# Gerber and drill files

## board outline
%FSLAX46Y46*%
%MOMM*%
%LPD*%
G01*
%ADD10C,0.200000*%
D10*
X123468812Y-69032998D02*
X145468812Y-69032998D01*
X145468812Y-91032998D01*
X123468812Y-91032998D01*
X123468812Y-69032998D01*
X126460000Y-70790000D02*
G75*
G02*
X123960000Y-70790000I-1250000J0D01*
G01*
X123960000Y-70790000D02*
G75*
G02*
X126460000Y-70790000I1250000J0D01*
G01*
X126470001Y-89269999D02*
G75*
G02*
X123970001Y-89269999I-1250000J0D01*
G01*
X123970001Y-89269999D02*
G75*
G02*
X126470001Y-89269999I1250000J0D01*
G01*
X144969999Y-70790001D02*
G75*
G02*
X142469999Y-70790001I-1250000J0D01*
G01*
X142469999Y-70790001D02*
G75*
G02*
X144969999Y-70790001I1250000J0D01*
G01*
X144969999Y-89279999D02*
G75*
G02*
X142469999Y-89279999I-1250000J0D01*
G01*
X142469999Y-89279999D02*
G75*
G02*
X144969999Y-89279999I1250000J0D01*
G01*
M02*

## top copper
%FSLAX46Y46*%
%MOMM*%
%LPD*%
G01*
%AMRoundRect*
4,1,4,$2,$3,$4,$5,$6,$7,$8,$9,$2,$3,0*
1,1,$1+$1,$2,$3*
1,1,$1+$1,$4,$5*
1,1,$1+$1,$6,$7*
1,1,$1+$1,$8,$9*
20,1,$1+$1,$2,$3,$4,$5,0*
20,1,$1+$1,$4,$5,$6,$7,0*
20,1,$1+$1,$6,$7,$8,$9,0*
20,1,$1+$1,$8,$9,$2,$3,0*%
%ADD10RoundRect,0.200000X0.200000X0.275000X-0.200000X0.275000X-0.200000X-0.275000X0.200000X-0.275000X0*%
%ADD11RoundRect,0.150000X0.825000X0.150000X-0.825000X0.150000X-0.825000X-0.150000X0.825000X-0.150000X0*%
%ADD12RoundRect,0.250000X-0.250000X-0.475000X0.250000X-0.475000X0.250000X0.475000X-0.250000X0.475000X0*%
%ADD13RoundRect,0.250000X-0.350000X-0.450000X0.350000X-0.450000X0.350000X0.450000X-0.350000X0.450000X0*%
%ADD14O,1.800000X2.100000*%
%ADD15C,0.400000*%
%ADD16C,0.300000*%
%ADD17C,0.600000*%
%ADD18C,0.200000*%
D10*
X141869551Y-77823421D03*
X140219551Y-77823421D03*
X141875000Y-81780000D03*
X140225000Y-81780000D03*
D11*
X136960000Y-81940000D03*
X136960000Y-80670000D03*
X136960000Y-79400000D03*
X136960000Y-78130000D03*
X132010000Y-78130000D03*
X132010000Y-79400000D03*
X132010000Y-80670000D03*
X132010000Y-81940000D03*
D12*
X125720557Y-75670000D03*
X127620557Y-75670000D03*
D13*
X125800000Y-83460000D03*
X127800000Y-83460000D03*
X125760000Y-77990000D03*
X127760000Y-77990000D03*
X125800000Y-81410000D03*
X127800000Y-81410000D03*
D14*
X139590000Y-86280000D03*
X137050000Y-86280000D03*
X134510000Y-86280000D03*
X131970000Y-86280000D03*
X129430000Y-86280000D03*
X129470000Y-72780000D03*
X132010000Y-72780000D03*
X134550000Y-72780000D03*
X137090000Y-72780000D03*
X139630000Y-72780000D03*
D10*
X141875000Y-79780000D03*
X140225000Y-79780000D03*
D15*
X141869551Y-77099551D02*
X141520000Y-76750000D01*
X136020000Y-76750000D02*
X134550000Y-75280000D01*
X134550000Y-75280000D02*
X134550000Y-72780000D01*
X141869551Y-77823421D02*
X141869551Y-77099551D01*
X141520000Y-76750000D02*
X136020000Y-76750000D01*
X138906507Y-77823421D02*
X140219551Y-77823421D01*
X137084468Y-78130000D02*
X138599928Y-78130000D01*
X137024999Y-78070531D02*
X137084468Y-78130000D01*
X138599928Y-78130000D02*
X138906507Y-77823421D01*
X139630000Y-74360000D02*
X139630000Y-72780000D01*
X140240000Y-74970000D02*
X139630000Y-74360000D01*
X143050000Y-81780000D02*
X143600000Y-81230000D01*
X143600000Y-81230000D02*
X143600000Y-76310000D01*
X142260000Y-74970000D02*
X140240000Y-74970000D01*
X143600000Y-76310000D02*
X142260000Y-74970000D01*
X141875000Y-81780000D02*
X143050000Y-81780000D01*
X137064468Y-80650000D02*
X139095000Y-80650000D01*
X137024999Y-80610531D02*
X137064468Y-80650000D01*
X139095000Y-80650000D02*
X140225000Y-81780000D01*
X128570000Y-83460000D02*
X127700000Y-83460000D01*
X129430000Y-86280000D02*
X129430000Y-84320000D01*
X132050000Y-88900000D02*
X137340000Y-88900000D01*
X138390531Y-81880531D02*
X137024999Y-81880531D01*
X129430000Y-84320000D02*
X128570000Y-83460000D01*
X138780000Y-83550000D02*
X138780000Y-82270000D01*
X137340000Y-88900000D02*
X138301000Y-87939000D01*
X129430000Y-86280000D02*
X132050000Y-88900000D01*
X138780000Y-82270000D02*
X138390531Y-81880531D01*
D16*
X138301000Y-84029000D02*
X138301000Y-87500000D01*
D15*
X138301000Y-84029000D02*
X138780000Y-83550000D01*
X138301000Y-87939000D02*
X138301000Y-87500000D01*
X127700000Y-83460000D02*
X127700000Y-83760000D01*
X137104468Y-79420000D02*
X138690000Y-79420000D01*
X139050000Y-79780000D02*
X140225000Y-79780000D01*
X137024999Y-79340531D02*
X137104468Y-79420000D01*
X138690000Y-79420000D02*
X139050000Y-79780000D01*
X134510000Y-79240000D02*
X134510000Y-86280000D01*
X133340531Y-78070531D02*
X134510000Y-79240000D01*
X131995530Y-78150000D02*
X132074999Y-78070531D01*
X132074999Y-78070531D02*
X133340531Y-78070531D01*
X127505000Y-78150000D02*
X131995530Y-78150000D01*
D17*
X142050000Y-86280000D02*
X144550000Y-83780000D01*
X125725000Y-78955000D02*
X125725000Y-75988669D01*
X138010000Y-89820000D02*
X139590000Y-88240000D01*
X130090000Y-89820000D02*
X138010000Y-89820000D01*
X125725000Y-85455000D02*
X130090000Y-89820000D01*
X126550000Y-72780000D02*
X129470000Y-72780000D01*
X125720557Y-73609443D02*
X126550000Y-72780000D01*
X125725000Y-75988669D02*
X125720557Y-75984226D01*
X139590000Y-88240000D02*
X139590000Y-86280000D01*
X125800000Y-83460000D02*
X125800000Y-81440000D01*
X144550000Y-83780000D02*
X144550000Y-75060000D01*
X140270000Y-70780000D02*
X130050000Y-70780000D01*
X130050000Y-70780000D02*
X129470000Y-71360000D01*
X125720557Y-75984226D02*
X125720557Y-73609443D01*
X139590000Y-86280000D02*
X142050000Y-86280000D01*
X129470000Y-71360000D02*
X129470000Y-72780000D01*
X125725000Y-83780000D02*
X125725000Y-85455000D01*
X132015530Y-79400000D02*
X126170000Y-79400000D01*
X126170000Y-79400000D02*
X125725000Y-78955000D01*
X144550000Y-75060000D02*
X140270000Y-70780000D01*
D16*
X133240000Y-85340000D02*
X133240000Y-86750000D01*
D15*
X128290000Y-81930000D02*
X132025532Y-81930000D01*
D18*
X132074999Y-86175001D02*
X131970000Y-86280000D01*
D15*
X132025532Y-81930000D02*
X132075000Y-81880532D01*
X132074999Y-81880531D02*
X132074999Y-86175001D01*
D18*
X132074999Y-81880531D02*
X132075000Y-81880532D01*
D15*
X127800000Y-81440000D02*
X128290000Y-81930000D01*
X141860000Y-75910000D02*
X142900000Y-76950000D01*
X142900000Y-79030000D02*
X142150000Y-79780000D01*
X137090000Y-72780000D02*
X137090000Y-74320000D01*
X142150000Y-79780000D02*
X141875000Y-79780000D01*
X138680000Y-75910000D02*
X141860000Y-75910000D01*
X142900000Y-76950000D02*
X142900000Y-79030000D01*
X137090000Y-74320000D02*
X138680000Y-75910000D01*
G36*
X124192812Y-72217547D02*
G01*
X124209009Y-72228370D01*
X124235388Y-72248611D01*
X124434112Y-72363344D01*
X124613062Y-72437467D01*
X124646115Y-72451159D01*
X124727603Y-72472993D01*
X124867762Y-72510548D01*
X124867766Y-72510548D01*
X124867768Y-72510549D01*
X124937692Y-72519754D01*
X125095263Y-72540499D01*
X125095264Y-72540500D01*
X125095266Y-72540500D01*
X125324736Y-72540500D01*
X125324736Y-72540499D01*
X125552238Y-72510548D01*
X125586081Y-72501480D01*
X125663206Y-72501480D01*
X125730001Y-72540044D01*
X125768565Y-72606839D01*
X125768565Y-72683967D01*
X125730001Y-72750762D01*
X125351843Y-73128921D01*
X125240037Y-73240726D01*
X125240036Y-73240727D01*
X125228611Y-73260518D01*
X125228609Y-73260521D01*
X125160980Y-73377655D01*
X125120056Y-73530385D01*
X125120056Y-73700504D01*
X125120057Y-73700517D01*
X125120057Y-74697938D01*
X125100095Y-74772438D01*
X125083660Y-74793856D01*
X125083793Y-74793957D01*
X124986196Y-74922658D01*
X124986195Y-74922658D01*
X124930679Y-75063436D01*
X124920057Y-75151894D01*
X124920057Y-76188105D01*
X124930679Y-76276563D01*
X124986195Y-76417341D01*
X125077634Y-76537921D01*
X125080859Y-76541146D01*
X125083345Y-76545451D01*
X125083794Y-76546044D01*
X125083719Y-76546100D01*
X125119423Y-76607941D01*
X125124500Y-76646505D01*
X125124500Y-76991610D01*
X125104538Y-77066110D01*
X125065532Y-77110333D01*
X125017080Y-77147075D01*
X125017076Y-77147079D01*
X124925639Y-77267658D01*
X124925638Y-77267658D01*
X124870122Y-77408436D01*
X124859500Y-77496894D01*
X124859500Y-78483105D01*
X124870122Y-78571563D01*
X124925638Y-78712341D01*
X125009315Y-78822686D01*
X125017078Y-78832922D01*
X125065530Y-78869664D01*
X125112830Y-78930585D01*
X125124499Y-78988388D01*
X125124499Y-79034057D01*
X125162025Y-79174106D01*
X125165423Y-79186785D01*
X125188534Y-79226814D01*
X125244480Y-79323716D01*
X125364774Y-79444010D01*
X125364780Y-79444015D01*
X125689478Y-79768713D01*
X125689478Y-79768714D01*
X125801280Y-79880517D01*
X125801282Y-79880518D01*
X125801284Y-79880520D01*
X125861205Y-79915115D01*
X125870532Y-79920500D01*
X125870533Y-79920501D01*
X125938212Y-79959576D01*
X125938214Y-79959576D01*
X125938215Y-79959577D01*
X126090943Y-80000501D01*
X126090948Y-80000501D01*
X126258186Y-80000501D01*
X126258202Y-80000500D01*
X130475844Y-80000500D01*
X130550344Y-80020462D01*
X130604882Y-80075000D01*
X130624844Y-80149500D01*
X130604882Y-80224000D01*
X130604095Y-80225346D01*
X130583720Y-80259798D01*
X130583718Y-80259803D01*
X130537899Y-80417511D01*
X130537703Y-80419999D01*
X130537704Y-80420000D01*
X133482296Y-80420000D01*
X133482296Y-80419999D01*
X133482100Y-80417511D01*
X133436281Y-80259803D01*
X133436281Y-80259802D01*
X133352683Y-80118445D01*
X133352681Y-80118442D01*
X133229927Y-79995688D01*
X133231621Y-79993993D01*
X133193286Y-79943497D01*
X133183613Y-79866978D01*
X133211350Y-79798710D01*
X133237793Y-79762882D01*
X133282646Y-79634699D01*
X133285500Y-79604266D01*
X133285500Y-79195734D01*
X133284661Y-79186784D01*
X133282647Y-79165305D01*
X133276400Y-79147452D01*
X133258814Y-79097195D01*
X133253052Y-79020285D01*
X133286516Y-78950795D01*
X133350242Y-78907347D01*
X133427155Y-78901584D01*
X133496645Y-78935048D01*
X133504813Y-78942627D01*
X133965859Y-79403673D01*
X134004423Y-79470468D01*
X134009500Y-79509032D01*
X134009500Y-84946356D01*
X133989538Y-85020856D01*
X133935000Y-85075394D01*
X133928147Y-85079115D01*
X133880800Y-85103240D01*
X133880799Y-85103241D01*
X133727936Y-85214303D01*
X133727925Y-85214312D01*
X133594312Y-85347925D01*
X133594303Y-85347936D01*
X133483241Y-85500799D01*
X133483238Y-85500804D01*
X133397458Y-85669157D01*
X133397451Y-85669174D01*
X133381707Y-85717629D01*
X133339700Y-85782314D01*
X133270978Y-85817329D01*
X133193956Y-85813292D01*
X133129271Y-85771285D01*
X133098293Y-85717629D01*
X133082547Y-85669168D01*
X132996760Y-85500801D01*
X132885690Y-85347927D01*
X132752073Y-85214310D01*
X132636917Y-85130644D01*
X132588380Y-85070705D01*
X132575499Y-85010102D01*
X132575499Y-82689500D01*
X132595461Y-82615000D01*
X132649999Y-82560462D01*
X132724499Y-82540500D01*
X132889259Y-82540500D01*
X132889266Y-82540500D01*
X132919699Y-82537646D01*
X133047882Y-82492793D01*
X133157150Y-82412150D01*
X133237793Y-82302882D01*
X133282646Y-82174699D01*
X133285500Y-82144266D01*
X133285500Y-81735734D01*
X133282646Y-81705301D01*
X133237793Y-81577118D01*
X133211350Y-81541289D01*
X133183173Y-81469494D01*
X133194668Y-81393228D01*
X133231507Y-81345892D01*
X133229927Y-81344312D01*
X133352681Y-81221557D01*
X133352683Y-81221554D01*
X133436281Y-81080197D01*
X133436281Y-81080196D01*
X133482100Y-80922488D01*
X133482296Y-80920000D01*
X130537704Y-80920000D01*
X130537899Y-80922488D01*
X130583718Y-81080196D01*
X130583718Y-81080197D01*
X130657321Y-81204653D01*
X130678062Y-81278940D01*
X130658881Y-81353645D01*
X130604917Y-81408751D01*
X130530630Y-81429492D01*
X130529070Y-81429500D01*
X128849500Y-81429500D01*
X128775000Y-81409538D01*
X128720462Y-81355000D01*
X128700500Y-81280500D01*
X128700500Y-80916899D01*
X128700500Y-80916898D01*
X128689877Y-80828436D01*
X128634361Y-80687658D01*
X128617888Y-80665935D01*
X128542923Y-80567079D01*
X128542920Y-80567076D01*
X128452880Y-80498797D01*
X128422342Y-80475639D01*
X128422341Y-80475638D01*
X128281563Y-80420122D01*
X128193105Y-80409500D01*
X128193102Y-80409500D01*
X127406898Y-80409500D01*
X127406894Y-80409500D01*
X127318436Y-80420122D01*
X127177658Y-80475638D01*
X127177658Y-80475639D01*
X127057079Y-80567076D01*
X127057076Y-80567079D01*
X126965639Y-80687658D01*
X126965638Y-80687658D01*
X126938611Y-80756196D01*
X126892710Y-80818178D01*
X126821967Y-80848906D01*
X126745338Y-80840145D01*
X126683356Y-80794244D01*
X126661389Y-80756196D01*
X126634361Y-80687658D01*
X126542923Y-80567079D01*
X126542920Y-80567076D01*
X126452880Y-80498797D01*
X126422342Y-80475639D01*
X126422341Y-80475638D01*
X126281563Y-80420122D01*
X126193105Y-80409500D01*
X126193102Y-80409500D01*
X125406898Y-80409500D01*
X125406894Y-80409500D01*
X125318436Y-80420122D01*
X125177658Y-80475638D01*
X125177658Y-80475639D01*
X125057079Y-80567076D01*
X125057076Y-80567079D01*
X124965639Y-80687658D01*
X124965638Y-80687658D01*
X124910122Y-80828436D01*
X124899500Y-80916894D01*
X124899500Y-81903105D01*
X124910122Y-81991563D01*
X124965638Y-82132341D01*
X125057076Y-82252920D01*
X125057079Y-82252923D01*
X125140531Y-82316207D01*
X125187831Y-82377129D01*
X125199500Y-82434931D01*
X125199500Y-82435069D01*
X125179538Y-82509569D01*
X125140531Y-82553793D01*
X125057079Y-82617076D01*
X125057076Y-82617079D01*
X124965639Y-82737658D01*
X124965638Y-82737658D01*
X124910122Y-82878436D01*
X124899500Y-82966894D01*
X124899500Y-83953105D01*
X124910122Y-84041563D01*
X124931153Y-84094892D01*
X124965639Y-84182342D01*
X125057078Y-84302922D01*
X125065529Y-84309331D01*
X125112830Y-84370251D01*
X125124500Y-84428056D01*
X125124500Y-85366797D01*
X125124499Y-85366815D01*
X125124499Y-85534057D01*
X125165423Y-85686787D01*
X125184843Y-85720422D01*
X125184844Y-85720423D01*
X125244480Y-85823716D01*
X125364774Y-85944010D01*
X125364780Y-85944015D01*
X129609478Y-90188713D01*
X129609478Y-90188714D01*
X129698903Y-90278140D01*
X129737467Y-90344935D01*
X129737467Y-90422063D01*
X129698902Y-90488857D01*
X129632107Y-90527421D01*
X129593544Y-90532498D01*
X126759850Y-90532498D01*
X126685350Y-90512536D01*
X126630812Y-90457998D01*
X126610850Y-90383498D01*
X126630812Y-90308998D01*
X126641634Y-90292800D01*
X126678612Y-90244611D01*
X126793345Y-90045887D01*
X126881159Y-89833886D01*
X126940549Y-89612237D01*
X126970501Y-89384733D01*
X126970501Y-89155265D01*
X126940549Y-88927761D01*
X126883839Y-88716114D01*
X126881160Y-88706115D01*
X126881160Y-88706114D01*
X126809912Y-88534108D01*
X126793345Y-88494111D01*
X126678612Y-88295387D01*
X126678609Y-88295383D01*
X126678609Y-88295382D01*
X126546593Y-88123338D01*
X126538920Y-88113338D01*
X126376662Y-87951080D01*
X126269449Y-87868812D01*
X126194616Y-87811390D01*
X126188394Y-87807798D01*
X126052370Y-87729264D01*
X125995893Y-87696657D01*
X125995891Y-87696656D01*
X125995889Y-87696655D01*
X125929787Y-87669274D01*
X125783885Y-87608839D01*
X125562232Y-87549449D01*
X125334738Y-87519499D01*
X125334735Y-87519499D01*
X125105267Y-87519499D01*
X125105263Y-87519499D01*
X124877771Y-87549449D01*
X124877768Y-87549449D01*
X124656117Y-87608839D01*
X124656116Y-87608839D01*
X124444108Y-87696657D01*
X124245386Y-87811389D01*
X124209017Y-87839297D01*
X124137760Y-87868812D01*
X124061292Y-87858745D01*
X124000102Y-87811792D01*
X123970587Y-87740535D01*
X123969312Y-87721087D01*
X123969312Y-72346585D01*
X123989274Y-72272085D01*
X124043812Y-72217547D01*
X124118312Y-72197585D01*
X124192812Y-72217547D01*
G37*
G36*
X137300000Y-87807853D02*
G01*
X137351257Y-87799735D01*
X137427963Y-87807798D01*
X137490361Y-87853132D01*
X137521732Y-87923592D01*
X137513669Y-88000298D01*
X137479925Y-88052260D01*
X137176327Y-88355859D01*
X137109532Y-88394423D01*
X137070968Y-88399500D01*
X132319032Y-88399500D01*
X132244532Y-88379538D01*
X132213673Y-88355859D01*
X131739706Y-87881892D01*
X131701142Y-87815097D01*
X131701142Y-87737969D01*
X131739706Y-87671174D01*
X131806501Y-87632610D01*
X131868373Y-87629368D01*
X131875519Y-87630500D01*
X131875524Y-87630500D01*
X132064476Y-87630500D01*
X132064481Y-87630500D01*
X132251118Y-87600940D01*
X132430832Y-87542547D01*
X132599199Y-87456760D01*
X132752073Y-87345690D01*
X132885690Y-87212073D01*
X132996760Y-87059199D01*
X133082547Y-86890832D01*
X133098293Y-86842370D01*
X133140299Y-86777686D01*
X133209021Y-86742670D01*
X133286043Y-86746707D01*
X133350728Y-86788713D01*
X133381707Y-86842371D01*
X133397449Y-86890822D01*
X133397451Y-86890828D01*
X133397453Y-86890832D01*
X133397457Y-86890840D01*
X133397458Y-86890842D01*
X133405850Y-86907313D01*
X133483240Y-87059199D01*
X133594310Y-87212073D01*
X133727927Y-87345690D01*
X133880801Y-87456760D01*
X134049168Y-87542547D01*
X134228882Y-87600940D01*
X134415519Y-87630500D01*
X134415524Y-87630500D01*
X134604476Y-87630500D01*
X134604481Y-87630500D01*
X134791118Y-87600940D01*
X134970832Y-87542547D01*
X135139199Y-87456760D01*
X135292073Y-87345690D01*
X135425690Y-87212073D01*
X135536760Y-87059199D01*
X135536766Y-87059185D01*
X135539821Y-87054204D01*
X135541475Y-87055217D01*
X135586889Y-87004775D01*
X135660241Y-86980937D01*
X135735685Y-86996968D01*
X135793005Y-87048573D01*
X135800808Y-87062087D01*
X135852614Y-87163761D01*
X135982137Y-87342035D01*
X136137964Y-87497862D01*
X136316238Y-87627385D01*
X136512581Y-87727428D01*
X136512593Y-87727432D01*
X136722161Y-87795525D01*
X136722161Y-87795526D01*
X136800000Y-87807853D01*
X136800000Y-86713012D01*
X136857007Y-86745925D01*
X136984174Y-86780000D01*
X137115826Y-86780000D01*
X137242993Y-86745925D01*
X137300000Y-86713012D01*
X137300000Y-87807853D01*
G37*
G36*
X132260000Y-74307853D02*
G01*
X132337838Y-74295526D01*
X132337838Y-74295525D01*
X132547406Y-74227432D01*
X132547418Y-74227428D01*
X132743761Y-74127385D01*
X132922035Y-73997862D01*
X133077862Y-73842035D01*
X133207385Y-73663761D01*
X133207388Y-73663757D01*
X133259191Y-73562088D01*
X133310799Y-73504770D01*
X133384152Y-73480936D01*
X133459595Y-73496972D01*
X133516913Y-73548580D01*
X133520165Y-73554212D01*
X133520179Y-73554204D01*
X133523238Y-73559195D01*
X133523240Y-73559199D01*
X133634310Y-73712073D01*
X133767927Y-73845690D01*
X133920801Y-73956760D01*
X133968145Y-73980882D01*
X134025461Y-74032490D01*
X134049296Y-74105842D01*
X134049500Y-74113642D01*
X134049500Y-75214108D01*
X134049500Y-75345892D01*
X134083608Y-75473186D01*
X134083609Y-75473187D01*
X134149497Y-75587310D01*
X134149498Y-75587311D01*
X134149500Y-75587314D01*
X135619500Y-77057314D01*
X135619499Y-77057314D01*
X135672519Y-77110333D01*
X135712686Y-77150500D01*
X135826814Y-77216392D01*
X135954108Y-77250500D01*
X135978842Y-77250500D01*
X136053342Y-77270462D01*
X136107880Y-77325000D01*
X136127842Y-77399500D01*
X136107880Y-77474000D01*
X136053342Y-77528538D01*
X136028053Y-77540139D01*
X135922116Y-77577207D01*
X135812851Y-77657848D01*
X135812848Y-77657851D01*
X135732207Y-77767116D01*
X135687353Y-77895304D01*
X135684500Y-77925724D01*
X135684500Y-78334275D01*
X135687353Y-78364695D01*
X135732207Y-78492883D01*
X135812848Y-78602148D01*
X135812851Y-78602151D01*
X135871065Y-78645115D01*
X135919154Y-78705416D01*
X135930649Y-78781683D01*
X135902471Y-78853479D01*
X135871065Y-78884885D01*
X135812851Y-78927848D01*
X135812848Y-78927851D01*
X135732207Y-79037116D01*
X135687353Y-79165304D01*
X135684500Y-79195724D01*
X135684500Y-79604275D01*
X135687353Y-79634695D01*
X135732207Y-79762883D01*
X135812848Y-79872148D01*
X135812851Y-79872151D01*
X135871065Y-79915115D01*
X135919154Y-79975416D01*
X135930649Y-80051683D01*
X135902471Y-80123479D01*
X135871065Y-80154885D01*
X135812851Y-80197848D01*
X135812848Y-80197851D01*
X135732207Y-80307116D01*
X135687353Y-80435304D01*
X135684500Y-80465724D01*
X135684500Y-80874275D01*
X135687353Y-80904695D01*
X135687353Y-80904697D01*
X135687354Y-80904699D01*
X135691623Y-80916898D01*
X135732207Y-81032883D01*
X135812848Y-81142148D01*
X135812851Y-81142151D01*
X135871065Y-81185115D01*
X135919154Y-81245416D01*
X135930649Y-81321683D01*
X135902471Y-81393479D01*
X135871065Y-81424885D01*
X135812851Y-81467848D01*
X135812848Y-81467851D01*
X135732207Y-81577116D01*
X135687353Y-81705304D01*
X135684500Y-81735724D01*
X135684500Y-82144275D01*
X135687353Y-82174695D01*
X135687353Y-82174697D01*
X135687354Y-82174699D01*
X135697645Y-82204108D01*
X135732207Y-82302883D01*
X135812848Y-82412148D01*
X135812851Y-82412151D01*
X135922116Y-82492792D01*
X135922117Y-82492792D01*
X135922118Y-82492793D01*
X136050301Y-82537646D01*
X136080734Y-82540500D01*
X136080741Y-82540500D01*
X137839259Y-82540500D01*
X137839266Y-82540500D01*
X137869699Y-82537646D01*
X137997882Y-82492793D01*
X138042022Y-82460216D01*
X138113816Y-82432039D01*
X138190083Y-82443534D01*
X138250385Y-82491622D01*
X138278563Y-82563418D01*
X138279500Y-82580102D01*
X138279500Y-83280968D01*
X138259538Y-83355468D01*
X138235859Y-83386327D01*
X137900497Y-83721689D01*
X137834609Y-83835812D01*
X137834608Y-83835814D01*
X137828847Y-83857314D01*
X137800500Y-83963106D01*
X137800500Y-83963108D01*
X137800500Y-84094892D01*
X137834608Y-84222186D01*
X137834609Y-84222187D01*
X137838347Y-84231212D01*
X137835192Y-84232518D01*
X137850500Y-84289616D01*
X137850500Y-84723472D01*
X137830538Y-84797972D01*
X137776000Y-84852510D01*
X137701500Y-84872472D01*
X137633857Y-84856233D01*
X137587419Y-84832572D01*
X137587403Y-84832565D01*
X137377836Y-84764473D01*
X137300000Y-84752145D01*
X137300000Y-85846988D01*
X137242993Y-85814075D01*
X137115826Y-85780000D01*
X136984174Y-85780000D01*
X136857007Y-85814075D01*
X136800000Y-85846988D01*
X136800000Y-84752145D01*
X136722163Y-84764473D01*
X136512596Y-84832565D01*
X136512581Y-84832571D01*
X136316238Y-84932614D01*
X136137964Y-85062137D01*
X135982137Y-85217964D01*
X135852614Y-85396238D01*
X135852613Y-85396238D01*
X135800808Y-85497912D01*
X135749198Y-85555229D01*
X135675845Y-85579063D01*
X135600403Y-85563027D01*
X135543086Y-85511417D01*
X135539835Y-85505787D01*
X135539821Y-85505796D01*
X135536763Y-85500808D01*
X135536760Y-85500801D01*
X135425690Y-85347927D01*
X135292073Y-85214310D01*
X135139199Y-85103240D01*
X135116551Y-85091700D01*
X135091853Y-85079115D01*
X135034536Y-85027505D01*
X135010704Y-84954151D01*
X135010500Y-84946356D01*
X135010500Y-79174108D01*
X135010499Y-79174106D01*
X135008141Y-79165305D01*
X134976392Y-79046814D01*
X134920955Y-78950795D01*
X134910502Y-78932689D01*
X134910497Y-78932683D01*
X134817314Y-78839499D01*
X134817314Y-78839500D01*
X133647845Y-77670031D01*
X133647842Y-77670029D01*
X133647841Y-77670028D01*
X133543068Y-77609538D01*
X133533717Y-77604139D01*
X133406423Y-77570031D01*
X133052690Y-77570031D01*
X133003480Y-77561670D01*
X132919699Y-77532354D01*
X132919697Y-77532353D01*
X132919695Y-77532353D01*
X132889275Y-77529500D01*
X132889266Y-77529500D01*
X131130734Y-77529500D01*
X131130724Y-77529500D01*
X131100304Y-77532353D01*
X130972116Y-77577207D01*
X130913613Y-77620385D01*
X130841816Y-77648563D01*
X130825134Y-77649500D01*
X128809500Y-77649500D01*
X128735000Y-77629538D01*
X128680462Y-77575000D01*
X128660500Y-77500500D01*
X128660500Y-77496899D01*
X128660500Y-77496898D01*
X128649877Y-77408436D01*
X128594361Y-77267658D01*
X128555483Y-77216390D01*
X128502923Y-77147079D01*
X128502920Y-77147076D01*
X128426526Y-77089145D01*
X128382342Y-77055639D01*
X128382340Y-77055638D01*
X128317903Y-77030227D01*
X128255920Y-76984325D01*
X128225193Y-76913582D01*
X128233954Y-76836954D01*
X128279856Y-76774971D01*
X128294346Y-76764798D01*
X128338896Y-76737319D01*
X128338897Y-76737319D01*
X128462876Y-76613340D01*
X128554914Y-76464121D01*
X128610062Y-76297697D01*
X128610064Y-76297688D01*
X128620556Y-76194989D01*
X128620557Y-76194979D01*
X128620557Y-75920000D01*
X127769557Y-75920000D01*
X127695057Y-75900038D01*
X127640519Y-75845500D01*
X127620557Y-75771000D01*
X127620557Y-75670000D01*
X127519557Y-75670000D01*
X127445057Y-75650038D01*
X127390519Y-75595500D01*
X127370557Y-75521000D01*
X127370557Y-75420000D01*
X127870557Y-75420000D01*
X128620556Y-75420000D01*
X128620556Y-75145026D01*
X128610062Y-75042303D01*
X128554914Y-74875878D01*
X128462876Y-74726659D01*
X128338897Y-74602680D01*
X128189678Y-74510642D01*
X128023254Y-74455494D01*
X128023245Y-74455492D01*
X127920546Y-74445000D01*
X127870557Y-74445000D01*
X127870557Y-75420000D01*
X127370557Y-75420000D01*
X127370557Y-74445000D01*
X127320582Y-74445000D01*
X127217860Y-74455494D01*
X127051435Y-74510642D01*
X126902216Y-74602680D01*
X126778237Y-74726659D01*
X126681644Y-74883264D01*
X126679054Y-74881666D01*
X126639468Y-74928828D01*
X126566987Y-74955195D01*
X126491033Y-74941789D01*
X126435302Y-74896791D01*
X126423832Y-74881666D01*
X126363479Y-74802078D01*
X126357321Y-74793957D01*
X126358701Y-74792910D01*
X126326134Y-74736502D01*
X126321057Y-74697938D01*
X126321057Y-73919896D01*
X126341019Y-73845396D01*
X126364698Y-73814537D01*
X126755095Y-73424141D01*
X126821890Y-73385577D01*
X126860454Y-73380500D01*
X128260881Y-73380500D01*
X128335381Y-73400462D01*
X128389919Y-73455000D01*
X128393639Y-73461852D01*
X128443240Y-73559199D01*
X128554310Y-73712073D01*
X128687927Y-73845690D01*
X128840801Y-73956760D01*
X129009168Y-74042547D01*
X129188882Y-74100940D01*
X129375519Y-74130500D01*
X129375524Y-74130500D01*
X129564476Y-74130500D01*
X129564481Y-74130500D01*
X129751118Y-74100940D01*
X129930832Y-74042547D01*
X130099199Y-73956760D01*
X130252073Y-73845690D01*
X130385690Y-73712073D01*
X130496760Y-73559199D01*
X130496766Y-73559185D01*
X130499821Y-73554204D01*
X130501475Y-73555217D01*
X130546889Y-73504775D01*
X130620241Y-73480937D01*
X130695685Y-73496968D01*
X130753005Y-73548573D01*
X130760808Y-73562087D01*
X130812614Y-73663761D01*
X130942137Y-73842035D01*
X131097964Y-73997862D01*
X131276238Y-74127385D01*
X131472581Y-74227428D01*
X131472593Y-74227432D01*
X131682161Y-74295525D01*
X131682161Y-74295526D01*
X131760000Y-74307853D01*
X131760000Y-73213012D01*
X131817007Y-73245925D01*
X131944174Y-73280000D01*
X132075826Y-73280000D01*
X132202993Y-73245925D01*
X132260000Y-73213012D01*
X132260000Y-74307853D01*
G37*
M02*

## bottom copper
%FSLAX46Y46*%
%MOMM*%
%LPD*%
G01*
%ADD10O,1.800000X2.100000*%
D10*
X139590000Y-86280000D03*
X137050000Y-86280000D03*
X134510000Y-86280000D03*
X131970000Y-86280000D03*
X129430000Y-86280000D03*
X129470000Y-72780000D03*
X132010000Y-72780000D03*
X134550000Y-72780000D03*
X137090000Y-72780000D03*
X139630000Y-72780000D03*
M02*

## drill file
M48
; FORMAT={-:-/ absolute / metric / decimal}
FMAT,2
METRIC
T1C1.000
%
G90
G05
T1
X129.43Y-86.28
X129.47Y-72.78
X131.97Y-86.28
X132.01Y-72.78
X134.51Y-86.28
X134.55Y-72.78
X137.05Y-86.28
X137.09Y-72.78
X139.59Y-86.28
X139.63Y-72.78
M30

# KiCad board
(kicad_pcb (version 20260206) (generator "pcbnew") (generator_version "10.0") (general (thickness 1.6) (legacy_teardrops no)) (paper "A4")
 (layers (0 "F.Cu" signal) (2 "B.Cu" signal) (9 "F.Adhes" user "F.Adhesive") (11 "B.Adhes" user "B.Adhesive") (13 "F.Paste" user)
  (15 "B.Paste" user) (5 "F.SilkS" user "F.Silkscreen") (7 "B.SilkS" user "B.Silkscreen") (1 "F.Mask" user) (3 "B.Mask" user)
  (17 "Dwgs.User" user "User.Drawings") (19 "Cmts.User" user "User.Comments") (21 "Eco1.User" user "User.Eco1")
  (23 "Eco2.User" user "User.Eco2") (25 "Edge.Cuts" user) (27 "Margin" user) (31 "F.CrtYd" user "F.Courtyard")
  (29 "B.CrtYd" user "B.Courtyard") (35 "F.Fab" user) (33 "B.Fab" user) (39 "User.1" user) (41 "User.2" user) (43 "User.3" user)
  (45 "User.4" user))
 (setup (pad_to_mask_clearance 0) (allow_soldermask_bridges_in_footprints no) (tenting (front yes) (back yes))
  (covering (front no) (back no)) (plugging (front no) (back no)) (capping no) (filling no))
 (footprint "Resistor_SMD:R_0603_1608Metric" (layer "F.Cu") (at 141.044551 77.823421 180)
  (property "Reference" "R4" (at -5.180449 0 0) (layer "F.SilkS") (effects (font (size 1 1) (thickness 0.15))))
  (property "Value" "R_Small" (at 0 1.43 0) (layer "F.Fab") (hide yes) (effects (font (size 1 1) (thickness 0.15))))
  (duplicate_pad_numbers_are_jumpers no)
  (pad "1" smd roundrect (at -0.825 0 180) (size 0.8 0.95) (layers "F.Cu" "F.Mask" "F.Paste") (roundrect_rratio 0.25) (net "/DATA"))
  (pad "2" smd roundrect (at 0.825 0 180) (size 0.8 0.95) (layers "F.Cu" "F.Mask" "F.Paste") (roundrect_rratio 0.25) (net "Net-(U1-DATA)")))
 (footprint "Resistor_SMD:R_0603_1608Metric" (layer "F.Cu") (at 141.05 81.78 180)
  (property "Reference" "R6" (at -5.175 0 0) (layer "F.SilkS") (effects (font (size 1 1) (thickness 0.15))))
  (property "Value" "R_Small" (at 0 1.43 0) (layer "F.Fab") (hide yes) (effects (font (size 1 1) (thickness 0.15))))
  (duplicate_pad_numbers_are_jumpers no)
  (pad "1" smd roundrect (at -0.825 0 180) (size 0.8 0.95) (layers "F.Cu" "F.Mask" "F.Paste") (roundrect_rratio 0.25) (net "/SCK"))
  (pad "2" smd roundrect (at 0.825 0 180) (size 0.8 0.95) (layers "F.Cu" "F.Mask" "F.Paste") (roundrect_rratio 0.25) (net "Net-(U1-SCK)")))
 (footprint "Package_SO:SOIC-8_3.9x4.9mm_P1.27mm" (layer "F.Cu") (at 134.485 80.035 180)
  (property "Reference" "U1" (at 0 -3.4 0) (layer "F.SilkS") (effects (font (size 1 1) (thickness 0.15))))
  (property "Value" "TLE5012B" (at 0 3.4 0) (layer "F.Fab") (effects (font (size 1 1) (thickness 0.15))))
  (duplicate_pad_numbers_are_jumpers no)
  (pad "1" smd roundrect (at -2.475 -1.905 180) (size 1.95 0.6) (layers "F.Cu" "F.Mask" "F.Paste") (roundrect_rratio 0.25) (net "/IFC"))
  (pad "2" smd roundrect (at -2.475 -0.635 180) (size 1.95 0.6) (layers "F.Cu" "F.Mask" "F.Paste") (roundrect_rratio 0.25)
   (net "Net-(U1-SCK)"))
  (pad "3" smd roundrect (at -2.475 0.635 180) (size 1.95 0.6) (layers "F.Cu" "F.Mask" "F.Paste") (roundrect_rratio 0.25)
   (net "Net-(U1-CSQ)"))
  (pad "4" smd roundrect (at -2.475 1.905 180) (size 1.95 0.6) (layers "F.Cu" "F.Mask" "F.Paste") (roundrect_rratio 0.25)
   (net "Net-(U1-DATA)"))
  (pad "5" smd roundrect (at 2.475 1.905 180) (size 1.95 0.6) (layers "F.Cu" "F.Mask" "F.Paste") (roundrect_rratio 0.25) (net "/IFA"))
  (pad "6" smd roundrect (at 2.475 0.635 180) (size 1.95 0.6) (layers "F.Cu" "F.Mask" "F.Paste") (roundrect_rratio 0.25) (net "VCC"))
  (pad "7" smd roundrect (at 2.475 -0.635 180) (size 1.95 0.6) (layers "F.Cu" "F.Mask" "F.Paste") (roundrect_rratio 0.25) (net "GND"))
  (pad "8" smd roundrect (at 2.475 -1.905 180) (size 1.95 0.6) (layers "F.Cu" "F.Mask" "F.Paste") (roundrect_rratio 0.25) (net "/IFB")))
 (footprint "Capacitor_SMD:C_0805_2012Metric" (layer "F.Cu") (at 126.670557 75.67)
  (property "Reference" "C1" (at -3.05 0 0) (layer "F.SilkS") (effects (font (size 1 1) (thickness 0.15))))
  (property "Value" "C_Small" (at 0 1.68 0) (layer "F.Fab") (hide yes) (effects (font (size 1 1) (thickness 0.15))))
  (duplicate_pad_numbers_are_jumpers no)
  (pad "1" smd roundrect (at -0.95 0) (size 1 1.45) (layers "F.Cu" "F.Mask" "F.Paste") (roundrect_rratio 0.25) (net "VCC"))
  (pad "2" smd roundrect (at 0.95 0) (size 1 1.45) (layers "F.Cu" "F.Mask" "F.Paste") (roundrect_rratio 0.25) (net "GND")))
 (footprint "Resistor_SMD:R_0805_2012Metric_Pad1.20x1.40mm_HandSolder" (layer "F.Cu") (at 126.8 83.46)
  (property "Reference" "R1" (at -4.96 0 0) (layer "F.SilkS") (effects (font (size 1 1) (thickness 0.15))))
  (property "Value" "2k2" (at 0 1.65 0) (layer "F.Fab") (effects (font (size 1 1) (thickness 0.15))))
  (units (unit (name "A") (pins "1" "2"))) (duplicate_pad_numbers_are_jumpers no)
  (pad "1" smd roundrect (at -1 0) (size 1.2 1.4) (layers "F.Cu" "F.Mask" "F.Paste") (roundrect_rratio 0.208333) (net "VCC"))
  (pad "2" smd roundrect (at 1 0) (size 1.2 1.4) (layers "F.Cu" "F.Mask" "F.Paste") (roundrect_rratio 0.208333) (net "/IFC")))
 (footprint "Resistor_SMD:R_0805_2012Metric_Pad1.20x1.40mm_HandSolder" (layer "F.Cu") (at 126.76 77.99)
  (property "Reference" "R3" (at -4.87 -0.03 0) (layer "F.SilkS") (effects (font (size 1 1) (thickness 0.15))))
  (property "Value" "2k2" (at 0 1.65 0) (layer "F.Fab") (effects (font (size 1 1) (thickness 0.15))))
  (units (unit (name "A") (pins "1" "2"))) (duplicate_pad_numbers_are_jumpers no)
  (pad "1" smd roundrect (at -1 0) (size 1.2 1.4) (layers "F.Cu" "F.Mask" "F.Paste") (roundrect_rratio 0.208333) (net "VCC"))
  (pad "2" smd roundrect (at 1 0) (size 1.2 1.4) (layers "F.Cu" "F.Mask" "F.Paste") (roundrect_rratio 0.208333) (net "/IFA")))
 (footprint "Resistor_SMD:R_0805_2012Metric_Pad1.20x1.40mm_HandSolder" (layer "F.Cu") (at 126.8 81.41)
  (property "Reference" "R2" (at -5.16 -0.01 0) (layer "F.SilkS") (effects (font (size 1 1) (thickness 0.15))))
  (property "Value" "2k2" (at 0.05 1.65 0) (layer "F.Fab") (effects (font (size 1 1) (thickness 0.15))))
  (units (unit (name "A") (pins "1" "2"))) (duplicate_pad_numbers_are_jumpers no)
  (pad "1" smd roundrect (at -1 0) (size 1.2 1.4) (layers "F.Cu" "F.Mask" "F.Paste") (roundrect_rratio 0.208333) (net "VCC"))
  (pad "2" smd roundrect (at 1 0) (size 1.2 1.4) (layers "F.Cu" "F.Mask" "F.Paste") (roundrect_rratio 0.208333) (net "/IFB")))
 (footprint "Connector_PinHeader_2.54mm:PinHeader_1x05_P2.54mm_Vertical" (layer "F.Cu") (at 139.59 86.28 -90)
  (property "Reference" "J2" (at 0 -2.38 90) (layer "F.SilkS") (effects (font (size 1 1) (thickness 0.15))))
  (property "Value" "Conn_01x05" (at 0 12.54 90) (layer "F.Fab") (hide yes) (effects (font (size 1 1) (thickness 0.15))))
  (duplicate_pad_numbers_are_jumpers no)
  (pad "1" thru_hole oval (at 0 0 270) (size 2.1 1.8) (drill 1) (layers "*.Cu" "*.Mask") (remove_unused_layers no) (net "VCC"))
  (pad "2" thru_hole oval (at 0 2.54 270) (size 2.1 1.8) (drill 1) (layers "*.Cu" "*.Mask") (remove_unused_layers no) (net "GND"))
  (pad "3" thru_hole oval (at 0 5.08 270) (size 2.1 1.8) (drill 1) (layers "*.Cu" "*.Mask") (remove_unused_layers no) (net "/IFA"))
  (pad "4" thru_hole oval (at 0 7.62 270) (size 2.1 1.8) (drill 1) (layers "*.Cu" "*.Mask") (remove_unused_layers no) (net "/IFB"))
  (pad "5" thru_hole oval (at 0 10.16 270) (size 2.1 1.8) (drill 1) (layers "*.Cu" "*.Mask") (remove_unused_layers no) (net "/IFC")))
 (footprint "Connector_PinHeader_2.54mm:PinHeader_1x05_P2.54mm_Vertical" (layer "F.Cu") (at 129.47 72.78 90)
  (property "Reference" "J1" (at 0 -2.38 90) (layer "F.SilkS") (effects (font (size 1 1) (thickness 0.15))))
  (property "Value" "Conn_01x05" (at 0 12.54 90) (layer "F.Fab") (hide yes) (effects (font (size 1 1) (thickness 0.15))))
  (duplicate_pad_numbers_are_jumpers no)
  (pad "1" thru_hole oval (at 0 0 90) (size 2.1 1.8) (drill 1) (layers "*.Cu" "*.Mask") (remove_unused_layers no) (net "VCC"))
  (pad "2" thru_hole oval (at 0 2.54 90) (size 2.1 1.8) (drill 1) (layers "*.Cu" "*.Mask") (remove_unused_layers no) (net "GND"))
  (pad "3" thru_hole oval (at 0 5.08 90) (size 2.1 1.8) (drill 1) (layers "*.Cu" "*.Mask") (remove_unused_layers no) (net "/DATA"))
  (pad "4" thru_hole oval (at 0 7.62 90) (size 2.1 1.8) (drill 1) (layers "*.Cu" "*.Mask") (remove_unused_layers no) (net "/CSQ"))
  (pad "5" thru_hole oval (at 0 10.16 90) (size 2.1 1.8) (drill 1) (layers "*.Cu" "*.Mask") (remove_unused_layers no) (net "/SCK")))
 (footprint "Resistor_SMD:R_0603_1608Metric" (layer "F.Cu") (at 141.05 79.78 180)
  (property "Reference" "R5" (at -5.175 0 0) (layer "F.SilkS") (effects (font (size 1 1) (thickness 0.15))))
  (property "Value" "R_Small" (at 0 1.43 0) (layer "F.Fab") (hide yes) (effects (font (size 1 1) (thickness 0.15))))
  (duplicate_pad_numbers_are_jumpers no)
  (pad "1" smd roundrect (at -0.825 0 180) (size 0.8 0.95) (layers "F.Cu" "F.Mask" "F.Paste") (roundrect_rratio 0.25) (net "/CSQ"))
  (pad "2" smd roundrect (at 0.825 0 180) (size 0.8 0.95) (layers "F.Cu" "F.Mask" "F.Paste") (roundrect_rratio 0.25) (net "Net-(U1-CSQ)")))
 (gr_rect (start 123.468812 69.032998) (end 145.468812 91.032998) (stroke (width 0.2) (type solid)) (fill no) (layer "Edge.Cuts"))
 (gr_circle (center 125.21 70.79) (end 125.209999 69.54) (stroke (width 0.2) (type solid)) (fill no) (layer "Edge.Cuts"))
 (gr_circle (center 125.220001 89.269999) (end 123.970001 89.27) (stroke (width 0.2) (type solid)) (fill no) (layer "Edge.Cuts"))
 (gr_circle (center 143.719999 70.790001) (end 144.969999 70.79) (stroke (width 0.2) (type solid)) (fill no) (layer "Edge.Cuts"))
 (gr_circle (center 143.719999 89.279999) (end 143.72 90.529999) (stroke (width 0.2) (type solid)) (fill no) (layer "Edge.Cuts"))
 (segment (start 141.869551 77.099551) (end 141.52 76.75) (width 0.4) (layer "F.Cu") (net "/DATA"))
 (segment (start 136.02 76.75) (end 134.55 75.28) (width 0.4) (layer "F.Cu") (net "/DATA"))
 (segment (start 134.55 75.28) (end 134.55 72.78) (width 0.4) (layer "F.Cu") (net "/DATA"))
 (segment (start 141.869551 77.823421) (end 141.869551 77.099551) (width 0.4) (layer "F.Cu") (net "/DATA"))
 (segment (start 141.52 76.75) (end 136.02 76.75) (width 0.4) (layer "F.Cu") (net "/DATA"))
 (segment (start 138.906507 77.823421) (end 140.219551 77.823421) (width 0.4) (layer "F.Cu") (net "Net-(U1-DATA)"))
 (segment (start 137.084468 78.13) (end 138.599928 78.13) (width 0.4) (layer "F.Cu") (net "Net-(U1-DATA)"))
 (segment (start 137.024999 78.070531) (end 137.084468 78.13) (width 0.4) (layer "F.Cu") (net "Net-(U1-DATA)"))
 (segment (start 138.599928 78.13) (end 138.906507 77.823421) (width 0.4) (layer "F.Cu") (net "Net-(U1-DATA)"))
 (segment (start 139.63 74.36) (end 139.63 72.78) (width 0.4) (layer "F.Cu") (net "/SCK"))
 (segment (start 140.24 74.97) (end 139.63 74.36) (width 0.4) (layer "F.Cu") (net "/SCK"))
 (segment (start 143.05 81.78) (end 143.6 81.23) (width 0.4) (layer "F.Cu") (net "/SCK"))
 (segment (start 143.6 81.23) (end 143.6 76.31) (width 0.4) (layer "F.Cu") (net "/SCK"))
 (segment (start 142.26 74.97) (end 140.24 74.97) (width 0.4) (layer "F.Cu") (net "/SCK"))
 (segment (start 143.6 76.31) (end 142.26 74.97) (width 0.4) (layer "F.Cu") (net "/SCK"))
 (segment (start 141.875 81.78) (end 143.05 81.78) (width 0.4) (layer "F.Cu") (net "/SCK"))
 (segment (start 137.064468 80.65) (end 139.095 80.65) (width 0.4) (layer "F.Cu") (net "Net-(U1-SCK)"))
 (segment (start 137.024999 80.610531) (end 137.064468 80.65) (width 0.4) (layer "F.Cu") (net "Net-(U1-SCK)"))
 (segment (start 139.095 80.65) (end 140.225 81.78) (width 0.4) (layer "F.Cu") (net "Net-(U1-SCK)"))
 (segment (start 128.57 83.46) (end 127.7 83.46) (width 0.4) (layer "F.Cu") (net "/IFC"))
 (segment (start 129.43 86.28) (end 129.43 84.32) (width 0.4) (layer "F.Cu") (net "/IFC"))
 (segment (start 132.05 88.9) (end 137.34 88.9) (width 0.4) (layer "F.Cu") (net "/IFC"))
 (segment (start 138.390531 81.880531) (end 137.024999 81.880531) (width 0.4) (layer "F.Cu") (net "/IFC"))
 (segment (start 129.43 84.32) (end 128.57 83.46) (width 0.4) (layer "F.Cu") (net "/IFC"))
 (segment (start 138.78 83.55) (end 138.78 82.27) (width 0.4) (layer "F.Cu") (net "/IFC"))
 (segment (start 137.34 88.9) (end 138.301 87.939) (width 0.4) (layer "F.Cu") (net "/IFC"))
 (segment (start 129.43 86.28) (end 132.05 88.9) (width 0.4) (layer "F.Cu") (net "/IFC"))
 (segment (start 138.78 82.27) (end 138.390531 81.880531) (width 0.4) (layer "F.Cu") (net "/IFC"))
 (segment (start 138.301 84.029) (end 138.301 87.5) (width 0.3) (layer "F.Cu") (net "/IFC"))
 (segment (start 138.301 84.029) (end 138.78 83.55) (width 0.4) (layer "F.Cu") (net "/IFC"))
 (segment (start 138.301 87.939) (end 138.301 87.5) (width 0.4) (layer "F.Cu") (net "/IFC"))
 (segment (start 127.7 83.46) (end 127.7 83.76) (width 0.4) (layer "F.Cu") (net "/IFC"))
 (segment (start 137.104468 79.42) (end 138.69 79.42) (width 0.4) (layer "F.Cu") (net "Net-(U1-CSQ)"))
 (segment (start 139.05 79.78) (end 140.225 79.78) (width 0.4) (layer "F.Cu") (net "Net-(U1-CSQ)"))
 (segment (start 137.024999 79.340531) (end 137.104468 79.42) (width 0.4) (layer "F.Cu") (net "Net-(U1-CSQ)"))
 (segment (start 138.69 79.42) (end 139.05 79.78) (width 0.4) (layer "F.Cu") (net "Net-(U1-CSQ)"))
 (segment (start 134.51 79.24) (end 134.51 86.28) (width 0.4) (layer "F.Cu") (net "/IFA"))
 (segment (start 133.340531 78.070531) (end 134.51 79.24) (width 0.4) (layer "F.Cu") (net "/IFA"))
 (segment (start 131.99553 78.15) (end 132.074999 78.070531) (width 0.4) (layer "F.Cu") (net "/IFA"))
 (segment (start 132.074999 78.070531) (end 133.340531 78.070531) (width 0.4) (layer "F.Cu") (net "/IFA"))
 (segment (start 127.505 78.15) (end 131.99553 78.15) (width 0.4) (layer "F.Cu") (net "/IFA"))
 (segment (start 142.05 86.28) (end 144.55 83.78) (width 0.6) (layer "F.Cu") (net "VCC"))
 (segment (start 125.725 78.955) (end 125.725 75.988669) (width 0.6) (layer "F.Cu") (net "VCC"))
 (segment (start 138.01 89.82) (end 139.59 88.24) (width 0.6) (layer "F.Cu") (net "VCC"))
 (segment (start 130.09 89.82) (end 138.01 89.82) (width 0.6) (layer "F.Cu") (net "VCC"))
 (segment (start 125.725 85.455) (end 130.09 89.82) (width 0.6) (layer "F.Cu") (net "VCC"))
 (segment (start 126.55 72.78) (end 129.47 72.78) (width 0.6) (layer "F.Cu") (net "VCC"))
 (segment (start 125.720557 73.609443) (end 126.55 72.78) (width 0.6) (layer "F.Cu") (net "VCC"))
 (segment (start 125.725 75.988669) (end 125.720557 75.984226) (width 0.6) (layer "F.Cu") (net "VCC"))
 (segment (start 139.59 88.24) (end 139.59 86.28) (width 0.6) (layer "F.Cu") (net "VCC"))
 (segment (start 125.8 83.46) (end 125.8 81.44) (width 0.6) (layer "F.Cu") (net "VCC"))
 (segment (start 144.55 83.78) (end 144.55 75.06) (width 0.6) (layer "F.Cu") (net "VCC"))
 (segment (start 140.27 70.78) (end 130.05 70.78) (width 0.6) (layer "F.Cu") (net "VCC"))
 (segment (start 130.05 70.78) (end 129.47 71.36) (width 0.6) (layer "F.Cu") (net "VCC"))
 (segment (start 125.720557 75.984226) (end 125.720557 73.609443) (width 0.6) (layer "F.Cu") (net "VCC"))
 (segment (start 139.59 86.28) (end 142.05 86.28) (width 0.6) (layer "F.Cu") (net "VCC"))
 (segment (start 129.47 71.36) (end 129.47 72.78) (width 0.6) (layer "F.Cu") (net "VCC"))
 (segment (start 125.725 83.78) (end 125.725 85.455) (width 0.6) (layer "F.Cu") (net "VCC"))
 (segment (start 132.01553 79.4) (end 126.17 79.4) (width 0.6) (layer "F.Cu") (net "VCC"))
 (segment (start 126.17 79.4) (end 125.725 78.955) (width 0.6) (layer "F.Cu") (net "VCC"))
 (segment (start 144.55 75.06) (end 140.27 70.78) (width 0.6) (layer "F.Cu") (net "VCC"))
 (segment (start 133.24 85.34) (end 133.24 86.75) (width 0.3) (layer "F.Cu") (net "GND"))
 (segment (start 128.29 81.93) (end 132.025532 81.93) (width 0.4) (layer "F.Cu") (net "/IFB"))
 (segment (start 132.074999 86.175001) (end 131.97 86.28) (width 0.2) (layer "F.Cu") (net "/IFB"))
 (segment (start 132.025532 81.93) (end 132.075 81.880532) (width 0.4) (layer "F.Cu") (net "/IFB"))
 (segment (start 132.074999 81.880531) (end 132.074999 86.175001) (width 0.4) (layer "F.Cu") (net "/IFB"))
 (segment (start 132.074999 81.880531) (end 132.075 81.880532) (width 0.2) (layer "F.Cu") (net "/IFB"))
 (segment (start 127.8 81.44) (end 128.29 81.93) (width 0.4) (layer "F.Cu") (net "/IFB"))
 (segment (start 141.86 75.91) (end 142.9 76.95) (width 0.4) (layer "F.Cu") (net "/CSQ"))
 (segment (start 142.9 79.03) (end 142.15 79.78) (width 0.4) (layer "F.Cu") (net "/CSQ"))
 (segment (start 137.09 72.78) (end 137.09 74.32) (width 0.4) (layer "F.Cu") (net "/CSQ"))
 (segment (start 142.15 79.78) (end 141.875 79.78) (width 0.4) (layer "F.Cu") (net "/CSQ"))
 (segment (start 138.68 75.91) (end 141.86 75.91) (width 0.4) (layer "F.Cu") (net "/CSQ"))
 (segment (start 142.9 76.95) (end 142.9 79.03) (width 0.4) (layer "F.Cu") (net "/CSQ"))
 (segment (start 137.09 74.32) (end 138.68 75.91) (width 0.4) (layer "F.Cu") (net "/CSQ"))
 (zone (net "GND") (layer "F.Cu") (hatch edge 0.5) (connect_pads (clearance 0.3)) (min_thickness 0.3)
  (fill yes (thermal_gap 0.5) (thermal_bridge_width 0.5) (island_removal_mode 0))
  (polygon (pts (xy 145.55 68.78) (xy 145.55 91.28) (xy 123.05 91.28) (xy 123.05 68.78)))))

